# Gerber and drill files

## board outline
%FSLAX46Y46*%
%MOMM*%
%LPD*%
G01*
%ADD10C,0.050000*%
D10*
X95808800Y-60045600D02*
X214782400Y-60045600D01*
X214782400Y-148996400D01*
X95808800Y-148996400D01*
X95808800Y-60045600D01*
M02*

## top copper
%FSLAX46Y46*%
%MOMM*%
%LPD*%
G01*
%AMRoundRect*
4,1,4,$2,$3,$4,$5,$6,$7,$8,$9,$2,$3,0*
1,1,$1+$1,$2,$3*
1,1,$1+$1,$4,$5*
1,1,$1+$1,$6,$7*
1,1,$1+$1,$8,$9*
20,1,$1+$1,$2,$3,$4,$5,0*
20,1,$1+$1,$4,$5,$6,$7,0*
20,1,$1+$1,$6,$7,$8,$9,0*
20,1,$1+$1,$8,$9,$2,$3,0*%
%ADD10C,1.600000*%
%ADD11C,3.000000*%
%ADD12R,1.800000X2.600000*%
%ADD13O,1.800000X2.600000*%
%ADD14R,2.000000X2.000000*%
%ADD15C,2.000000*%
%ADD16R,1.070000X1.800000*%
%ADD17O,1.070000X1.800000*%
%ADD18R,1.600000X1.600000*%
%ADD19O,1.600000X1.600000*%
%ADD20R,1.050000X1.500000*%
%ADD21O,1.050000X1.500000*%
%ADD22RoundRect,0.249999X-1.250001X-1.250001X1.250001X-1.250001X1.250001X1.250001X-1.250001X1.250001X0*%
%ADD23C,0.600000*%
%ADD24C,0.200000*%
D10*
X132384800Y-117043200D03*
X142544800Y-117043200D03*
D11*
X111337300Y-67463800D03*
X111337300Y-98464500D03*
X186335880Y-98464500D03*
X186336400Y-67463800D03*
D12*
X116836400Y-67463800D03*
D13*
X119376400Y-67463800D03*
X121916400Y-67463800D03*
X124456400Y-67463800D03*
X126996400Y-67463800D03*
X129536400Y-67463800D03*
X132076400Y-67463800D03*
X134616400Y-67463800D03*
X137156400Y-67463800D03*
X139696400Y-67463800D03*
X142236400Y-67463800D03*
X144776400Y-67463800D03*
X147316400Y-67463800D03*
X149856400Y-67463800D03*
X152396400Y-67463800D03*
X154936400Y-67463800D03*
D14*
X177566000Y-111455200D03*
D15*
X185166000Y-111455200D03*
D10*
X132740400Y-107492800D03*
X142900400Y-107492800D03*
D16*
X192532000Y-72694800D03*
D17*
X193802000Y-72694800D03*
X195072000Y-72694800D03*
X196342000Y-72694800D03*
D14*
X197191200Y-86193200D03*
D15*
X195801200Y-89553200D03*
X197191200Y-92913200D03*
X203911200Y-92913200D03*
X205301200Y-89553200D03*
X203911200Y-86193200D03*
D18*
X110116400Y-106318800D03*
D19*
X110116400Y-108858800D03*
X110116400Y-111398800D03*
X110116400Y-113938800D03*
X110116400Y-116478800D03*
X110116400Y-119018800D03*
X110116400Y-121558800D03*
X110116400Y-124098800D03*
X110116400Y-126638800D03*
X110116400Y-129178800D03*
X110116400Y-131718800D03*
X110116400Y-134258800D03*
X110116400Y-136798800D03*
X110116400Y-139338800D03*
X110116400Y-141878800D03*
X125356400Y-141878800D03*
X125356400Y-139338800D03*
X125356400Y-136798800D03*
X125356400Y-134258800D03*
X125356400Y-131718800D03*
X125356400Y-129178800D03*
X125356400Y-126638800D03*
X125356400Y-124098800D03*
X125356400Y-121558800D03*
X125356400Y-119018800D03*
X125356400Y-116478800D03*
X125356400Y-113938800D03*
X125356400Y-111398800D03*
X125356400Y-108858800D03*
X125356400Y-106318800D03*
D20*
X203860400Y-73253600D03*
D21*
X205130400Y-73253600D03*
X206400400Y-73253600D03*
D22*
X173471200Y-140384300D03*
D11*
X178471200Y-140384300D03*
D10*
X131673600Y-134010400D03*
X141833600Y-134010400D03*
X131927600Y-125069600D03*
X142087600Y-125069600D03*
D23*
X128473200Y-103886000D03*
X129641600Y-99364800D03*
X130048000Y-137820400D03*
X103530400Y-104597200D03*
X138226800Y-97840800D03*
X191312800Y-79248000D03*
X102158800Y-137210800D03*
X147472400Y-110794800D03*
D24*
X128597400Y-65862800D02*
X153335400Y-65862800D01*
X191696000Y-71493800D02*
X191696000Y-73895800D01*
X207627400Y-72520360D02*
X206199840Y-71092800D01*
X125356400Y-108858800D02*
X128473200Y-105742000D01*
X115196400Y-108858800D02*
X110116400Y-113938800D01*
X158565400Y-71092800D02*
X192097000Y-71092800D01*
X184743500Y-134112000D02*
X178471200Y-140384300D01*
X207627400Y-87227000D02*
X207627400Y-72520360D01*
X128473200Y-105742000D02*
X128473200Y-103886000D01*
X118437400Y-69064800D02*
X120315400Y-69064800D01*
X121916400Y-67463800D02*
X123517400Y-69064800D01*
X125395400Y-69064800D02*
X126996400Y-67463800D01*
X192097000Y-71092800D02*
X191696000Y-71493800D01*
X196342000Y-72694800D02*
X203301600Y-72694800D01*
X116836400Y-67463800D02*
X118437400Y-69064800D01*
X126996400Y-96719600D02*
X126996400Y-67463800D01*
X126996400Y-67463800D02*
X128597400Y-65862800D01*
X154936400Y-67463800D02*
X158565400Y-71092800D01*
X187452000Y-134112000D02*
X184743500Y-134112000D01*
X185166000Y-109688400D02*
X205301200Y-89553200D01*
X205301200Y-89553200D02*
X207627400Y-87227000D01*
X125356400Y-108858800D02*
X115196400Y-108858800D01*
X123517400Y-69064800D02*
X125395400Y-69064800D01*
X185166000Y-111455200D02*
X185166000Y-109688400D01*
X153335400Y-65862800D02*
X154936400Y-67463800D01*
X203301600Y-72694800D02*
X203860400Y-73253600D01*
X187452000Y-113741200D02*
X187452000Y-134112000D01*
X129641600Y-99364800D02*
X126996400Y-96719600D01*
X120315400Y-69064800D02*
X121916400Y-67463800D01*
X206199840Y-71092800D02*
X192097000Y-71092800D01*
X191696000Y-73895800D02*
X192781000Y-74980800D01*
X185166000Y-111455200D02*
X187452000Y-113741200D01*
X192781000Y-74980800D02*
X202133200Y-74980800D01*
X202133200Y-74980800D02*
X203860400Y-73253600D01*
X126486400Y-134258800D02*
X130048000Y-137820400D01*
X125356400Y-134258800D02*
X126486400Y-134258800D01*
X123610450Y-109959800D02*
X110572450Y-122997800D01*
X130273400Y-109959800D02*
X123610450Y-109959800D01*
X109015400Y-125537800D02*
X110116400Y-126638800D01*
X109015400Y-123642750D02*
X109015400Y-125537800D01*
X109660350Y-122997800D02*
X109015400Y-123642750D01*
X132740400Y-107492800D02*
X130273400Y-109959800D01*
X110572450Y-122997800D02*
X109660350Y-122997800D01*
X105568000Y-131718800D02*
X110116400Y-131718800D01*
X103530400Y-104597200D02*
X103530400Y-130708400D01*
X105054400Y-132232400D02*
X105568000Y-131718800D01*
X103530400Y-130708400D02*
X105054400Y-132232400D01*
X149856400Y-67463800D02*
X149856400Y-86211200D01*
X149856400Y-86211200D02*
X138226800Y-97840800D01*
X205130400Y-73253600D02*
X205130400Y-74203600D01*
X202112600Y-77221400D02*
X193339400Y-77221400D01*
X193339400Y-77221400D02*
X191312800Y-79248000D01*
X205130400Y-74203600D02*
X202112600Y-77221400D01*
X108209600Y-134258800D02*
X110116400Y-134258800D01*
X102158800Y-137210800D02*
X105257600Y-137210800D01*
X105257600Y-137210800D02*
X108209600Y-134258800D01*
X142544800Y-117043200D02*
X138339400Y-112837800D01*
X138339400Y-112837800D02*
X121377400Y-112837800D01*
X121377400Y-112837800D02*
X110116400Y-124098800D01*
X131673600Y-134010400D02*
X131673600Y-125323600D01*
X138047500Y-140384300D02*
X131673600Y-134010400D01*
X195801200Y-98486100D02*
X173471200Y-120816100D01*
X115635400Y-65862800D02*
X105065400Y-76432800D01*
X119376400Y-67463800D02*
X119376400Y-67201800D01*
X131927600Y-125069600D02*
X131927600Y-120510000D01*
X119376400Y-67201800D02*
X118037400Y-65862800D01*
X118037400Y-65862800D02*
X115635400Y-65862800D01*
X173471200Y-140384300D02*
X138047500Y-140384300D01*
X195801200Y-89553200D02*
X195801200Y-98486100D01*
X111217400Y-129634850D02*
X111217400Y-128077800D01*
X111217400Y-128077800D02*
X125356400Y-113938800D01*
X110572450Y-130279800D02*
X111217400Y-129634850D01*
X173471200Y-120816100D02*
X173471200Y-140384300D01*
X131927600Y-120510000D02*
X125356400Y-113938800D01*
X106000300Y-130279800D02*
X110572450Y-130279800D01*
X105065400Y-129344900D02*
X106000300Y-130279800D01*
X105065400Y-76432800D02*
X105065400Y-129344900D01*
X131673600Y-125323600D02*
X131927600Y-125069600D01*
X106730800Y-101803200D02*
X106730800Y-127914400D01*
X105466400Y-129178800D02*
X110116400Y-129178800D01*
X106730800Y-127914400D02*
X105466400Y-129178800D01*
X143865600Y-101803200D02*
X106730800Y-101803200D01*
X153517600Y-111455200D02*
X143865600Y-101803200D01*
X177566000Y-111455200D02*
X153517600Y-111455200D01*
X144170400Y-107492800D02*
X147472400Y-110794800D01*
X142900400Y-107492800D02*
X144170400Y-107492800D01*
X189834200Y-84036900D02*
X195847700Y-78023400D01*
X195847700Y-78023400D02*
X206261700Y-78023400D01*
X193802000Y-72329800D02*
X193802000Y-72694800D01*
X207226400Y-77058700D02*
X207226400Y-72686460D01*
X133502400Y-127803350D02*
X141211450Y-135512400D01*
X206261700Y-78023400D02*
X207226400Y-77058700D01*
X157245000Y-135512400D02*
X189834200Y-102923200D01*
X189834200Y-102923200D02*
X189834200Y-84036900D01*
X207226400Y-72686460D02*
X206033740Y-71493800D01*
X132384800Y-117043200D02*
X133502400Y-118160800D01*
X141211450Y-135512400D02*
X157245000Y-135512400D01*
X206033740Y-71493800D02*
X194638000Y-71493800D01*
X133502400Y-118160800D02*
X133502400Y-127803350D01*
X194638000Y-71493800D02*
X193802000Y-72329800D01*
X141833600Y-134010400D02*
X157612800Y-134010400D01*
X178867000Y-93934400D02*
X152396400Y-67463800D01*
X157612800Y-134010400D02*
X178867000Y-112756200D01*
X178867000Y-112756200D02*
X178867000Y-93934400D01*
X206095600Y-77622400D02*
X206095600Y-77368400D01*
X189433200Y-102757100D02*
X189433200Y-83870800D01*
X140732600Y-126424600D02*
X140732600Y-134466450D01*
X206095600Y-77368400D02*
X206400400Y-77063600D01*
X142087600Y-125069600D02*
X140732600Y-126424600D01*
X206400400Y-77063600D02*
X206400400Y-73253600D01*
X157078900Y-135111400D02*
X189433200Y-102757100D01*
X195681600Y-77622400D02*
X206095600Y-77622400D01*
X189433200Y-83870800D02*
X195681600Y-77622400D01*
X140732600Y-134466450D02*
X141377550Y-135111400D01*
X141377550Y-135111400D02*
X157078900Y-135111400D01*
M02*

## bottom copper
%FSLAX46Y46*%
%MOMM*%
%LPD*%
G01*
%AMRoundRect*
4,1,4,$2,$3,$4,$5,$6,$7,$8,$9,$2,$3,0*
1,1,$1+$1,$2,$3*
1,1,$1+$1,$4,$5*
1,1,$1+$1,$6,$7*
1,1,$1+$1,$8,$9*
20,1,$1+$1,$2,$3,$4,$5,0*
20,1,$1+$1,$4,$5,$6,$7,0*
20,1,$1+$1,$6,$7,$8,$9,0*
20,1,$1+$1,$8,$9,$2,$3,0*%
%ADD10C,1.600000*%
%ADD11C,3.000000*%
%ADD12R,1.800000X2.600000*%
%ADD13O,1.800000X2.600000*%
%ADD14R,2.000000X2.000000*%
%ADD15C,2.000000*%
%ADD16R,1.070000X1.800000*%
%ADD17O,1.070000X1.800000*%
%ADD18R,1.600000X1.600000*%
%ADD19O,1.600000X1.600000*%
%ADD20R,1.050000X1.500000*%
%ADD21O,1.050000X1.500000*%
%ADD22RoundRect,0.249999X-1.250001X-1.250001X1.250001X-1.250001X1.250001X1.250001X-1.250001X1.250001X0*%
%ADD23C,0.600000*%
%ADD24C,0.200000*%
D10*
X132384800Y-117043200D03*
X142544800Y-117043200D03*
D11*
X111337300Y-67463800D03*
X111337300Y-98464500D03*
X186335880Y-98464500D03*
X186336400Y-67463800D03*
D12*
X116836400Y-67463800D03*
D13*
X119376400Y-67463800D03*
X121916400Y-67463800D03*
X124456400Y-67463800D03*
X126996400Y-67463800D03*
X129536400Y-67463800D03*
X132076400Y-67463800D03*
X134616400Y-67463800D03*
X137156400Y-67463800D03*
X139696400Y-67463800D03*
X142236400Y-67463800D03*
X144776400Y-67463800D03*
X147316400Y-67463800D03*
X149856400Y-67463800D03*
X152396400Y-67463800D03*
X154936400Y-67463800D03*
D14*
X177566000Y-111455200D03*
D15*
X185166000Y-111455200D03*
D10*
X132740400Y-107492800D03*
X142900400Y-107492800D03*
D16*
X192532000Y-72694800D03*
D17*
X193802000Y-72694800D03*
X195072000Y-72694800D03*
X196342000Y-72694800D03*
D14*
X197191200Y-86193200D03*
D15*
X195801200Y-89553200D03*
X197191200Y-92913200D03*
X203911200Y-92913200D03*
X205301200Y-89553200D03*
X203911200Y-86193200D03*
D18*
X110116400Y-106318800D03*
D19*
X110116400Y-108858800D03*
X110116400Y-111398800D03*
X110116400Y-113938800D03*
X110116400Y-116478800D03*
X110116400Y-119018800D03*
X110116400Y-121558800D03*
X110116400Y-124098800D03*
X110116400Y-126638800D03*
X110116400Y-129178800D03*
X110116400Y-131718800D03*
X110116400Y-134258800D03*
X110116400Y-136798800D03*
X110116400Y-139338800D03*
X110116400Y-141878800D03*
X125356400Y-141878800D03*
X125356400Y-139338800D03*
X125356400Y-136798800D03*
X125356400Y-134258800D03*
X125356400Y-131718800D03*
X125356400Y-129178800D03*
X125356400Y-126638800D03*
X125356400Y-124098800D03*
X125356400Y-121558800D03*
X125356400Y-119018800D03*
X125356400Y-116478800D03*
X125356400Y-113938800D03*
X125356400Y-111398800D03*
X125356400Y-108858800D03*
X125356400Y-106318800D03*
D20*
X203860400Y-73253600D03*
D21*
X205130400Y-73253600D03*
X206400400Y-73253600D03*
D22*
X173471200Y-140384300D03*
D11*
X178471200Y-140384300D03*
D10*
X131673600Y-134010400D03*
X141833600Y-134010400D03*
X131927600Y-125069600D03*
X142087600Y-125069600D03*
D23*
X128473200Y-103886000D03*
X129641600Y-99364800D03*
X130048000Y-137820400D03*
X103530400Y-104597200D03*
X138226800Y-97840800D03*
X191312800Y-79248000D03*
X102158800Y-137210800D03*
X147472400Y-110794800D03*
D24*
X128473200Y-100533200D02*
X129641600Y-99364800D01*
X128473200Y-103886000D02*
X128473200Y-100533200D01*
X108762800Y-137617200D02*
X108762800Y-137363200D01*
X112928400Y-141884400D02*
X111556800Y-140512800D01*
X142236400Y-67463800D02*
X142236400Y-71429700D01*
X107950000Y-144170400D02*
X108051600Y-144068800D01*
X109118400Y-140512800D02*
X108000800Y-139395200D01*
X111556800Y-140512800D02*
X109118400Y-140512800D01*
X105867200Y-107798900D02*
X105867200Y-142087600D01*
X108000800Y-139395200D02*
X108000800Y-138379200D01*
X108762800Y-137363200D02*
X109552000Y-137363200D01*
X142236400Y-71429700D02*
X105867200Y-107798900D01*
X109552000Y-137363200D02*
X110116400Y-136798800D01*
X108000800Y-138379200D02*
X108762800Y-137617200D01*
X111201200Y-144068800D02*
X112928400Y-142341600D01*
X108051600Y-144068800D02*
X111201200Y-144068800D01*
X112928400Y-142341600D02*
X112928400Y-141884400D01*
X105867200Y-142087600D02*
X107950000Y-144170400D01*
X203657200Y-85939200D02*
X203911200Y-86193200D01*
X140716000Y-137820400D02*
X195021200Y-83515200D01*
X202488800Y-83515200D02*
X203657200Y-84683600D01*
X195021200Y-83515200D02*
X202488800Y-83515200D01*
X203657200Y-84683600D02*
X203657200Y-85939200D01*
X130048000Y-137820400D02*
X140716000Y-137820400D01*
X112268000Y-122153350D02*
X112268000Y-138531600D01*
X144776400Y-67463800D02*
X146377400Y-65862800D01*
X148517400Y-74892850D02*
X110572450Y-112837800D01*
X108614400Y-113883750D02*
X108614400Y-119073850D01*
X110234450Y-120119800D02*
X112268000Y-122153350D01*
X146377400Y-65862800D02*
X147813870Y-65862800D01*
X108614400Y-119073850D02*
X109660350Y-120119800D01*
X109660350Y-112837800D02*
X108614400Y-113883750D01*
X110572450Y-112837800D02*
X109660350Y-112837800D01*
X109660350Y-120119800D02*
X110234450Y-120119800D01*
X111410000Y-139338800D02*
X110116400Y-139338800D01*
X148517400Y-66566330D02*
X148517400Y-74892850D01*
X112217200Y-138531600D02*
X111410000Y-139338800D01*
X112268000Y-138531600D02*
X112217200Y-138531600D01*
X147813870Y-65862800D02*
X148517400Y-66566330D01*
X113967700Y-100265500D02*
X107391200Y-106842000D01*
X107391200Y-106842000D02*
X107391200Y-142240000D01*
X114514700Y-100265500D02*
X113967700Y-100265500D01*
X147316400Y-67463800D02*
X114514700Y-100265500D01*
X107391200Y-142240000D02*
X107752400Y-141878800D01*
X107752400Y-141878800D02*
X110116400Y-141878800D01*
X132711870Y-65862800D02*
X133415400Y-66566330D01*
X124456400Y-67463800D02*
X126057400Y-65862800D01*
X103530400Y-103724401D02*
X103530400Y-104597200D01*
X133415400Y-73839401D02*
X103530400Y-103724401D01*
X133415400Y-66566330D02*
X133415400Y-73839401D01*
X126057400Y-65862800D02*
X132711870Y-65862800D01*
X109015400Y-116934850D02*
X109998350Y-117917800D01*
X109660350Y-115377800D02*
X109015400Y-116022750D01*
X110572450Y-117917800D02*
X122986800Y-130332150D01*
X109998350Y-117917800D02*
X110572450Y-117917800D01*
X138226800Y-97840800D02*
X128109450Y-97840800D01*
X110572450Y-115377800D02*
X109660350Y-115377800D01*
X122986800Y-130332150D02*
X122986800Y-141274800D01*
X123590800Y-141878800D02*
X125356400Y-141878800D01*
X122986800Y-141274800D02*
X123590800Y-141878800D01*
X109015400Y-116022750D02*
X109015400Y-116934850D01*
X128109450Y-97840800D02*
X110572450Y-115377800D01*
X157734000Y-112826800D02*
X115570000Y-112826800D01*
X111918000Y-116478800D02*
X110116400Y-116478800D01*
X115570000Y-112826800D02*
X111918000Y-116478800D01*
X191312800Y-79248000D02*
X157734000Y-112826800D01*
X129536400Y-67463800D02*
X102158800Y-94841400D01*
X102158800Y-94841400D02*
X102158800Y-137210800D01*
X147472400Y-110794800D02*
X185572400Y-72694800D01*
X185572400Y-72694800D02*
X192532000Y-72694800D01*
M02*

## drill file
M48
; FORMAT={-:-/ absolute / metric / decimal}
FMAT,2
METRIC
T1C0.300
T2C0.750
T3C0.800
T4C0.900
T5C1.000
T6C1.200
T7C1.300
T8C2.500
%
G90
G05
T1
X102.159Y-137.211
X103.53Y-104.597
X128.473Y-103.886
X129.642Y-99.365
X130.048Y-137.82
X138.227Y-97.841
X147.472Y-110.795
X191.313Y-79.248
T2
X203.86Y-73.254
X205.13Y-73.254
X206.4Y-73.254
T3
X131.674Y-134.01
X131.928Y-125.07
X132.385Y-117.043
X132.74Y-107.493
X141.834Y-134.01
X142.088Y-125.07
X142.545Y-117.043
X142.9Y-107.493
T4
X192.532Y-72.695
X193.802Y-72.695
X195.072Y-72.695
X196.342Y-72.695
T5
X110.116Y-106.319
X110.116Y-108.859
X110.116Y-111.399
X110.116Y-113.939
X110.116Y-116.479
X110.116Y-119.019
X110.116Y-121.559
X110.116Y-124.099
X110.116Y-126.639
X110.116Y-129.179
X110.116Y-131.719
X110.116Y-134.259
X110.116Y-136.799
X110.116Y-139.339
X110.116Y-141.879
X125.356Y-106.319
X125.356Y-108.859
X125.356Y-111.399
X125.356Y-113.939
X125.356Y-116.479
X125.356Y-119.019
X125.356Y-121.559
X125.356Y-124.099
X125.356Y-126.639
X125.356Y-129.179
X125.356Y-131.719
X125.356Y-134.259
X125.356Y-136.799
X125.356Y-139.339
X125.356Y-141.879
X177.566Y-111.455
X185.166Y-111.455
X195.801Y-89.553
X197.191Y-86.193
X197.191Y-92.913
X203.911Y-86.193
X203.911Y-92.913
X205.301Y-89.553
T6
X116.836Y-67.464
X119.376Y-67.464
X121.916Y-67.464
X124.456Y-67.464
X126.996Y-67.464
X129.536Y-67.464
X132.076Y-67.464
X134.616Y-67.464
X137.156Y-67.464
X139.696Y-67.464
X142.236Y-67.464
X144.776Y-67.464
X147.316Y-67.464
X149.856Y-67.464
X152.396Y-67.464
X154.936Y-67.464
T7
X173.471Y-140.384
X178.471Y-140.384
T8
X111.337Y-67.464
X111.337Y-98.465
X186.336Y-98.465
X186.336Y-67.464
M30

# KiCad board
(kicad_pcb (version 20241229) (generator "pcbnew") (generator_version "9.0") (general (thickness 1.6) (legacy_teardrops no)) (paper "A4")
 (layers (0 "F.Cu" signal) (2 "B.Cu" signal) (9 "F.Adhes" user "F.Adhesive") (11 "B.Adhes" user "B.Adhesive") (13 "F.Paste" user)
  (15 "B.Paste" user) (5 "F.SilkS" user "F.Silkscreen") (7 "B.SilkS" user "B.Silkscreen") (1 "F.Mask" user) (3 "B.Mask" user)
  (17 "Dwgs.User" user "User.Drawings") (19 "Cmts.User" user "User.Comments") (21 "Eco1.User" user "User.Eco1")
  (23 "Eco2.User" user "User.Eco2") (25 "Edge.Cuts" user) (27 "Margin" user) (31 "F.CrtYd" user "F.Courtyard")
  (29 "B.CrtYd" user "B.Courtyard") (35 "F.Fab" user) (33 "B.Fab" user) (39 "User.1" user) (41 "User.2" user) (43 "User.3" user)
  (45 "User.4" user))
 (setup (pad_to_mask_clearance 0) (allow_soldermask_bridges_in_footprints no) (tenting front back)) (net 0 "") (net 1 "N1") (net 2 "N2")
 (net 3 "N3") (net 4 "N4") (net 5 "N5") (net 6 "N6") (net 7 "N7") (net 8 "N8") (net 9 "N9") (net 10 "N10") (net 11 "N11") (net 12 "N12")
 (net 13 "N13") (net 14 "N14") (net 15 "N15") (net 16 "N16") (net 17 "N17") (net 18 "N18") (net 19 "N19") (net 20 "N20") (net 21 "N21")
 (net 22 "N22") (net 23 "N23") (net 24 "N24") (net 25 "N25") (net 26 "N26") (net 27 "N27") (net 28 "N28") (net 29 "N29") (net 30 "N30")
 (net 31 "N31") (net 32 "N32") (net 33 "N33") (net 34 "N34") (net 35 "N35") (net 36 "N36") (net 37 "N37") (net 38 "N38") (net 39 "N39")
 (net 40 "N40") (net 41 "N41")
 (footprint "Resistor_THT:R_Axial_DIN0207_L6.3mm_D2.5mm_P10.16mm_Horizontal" (layer "F.Cu") (at 132.3848 117.0432)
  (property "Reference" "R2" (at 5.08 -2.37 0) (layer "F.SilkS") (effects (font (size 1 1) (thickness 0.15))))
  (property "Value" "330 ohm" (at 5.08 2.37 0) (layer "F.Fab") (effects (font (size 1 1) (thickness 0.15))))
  (pad "1" thru_hole circle (at 0 0) (size 1.6 1.6) (drill 0.8) (layers "*.Cu" "*.Mask") (remove_unused_layers no) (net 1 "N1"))
  (pad "2" thru_hole circle (at 10.16 0) (size 1.6 1.6) (drill 0.8) (layers "*.Cu" "*.Mask") (remove_unused_layers no) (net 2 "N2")))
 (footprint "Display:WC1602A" (layer "F.Cu") (at 116.8364 67.4638)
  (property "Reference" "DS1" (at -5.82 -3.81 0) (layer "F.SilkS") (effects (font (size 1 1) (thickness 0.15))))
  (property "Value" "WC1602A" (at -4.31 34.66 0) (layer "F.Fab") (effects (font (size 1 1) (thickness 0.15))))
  (pad "" thru_hole circle (at -5.4991 0) (size 3 3) (drill 2.5) (layers "*.Cu" "*.Mask") (remove_unused_layers no))
  (pad "" thru_hole circle (at -5.4991 31.0007) (size 3 3) (drill 2.5) (layers "*.Cu" "*.Mask") (remove_unused_layers no))
  (pad "" thru_hole circle (at 69.49948 31.0007) (size 3 3) (drill 2.5) (layers "*.Cu" "*.Mask") (remove_unused_layers no))
  (pad "" thru_hole circle (at 69.5 0) (size 3 3) (drill 2.5) (layers "*.Cu" "*.Mask") (remove_unused_layers no))
  (pad "1" thru_hole rect (at 0 0) (size 1.8 2.6) (drill 1.2) (layers "*.Cu" "*.Mask") (remove_unused_layers no) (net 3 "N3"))
  (pad "2" thru_hole oval (at 2.54 0) (size 1.8 2.6) (drill 1.2) (layers "*.Cu" "*.Mask") (remove_unused_layers no) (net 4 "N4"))
  (pad "3" thru_hole oval (at 5.08 0) (size 1.8 2.6) (drill 1.2) (layers "*.Cu" "*.Mask") (remove_unused_layers no) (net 3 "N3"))
  (pad "4" thru_hole oval (at 7.62 0) (size 1.8 2.6) (drill 1.2) (layers "*.Cu" "*.Mask") (remove_unused_layers no) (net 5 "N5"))
  (pad "5" thru_hole oval (at 10.16 0) (size 1.8 2.6) (drill 1.2) (layers "*.Cu" "*.Mask") (remove_unused_layers no) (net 3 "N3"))
  (pad "6" thru_hole oval (at 12.7 0) (size 1.8 2.6) (drill 1.2) (layers "*.Cu" "*.Mask") (remove_unused_layers no) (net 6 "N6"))
  (pad "7" thru_hole oval (at 15.24 0) (size 1.8 2.6) (drill 1.2) (layers "*.Cu" "*.Mask") (remove_unused_layers no) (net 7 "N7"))
  (pad "8" thru_hole oval (at 17.78 0) (size 1.8 2.6) (drill 1.2) (layers "*.Cu" "*.Mask") (remove_unused_layers no) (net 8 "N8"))
  (pad "9" thru_hole oval (at 20.32 0) (size 1.8 2.6) (drill 1.2) (layers "*.Cu" "*.Mask") (remove_unused_layers no) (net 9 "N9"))
  (pad "10" thru_hole oval (at 22.86 0) (size 1.8 2.6) (drill 1.2) (layers "*.Cu" "*.Mask") (remove_unused_layers no) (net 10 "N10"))
  (pad "11" thru_hole oval (at 25.4 0) (size 1.8 2.6) (drill 1.2) (layers "*.Cu" "*.Mask") (remove_unused_layers no) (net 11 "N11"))
  (pad "12" thru_hole oval (at 27.94 0) (size 1.8 2.6) (drill 1.2) (layers "*.Cu" "*.Mask") (remove_unused_layers no) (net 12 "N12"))
  (pad "13" thru_hole oval (at 30.48 0) (size 1.8 2.6) (drill 1.2) (layers "*.Cu" "*.Mask") (remove_unused_layers no) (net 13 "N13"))
  (pad "14" thru_hole oval (at 33.02 0) (size 1.8 2.6) (drill 1.2) (layers "*.Cu" "*.Mask") (remove_unused_layers no) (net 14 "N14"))
  (pad "15" thru_hole oval (at 35.56 0) (size 1.8 2.6) (drill 1.2) (layers "*.Cu" "*.Mask") (remove_unused_layers no) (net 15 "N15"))
  (pad "16" thru_hole oval (at 38.1 0) (size 1.8 2.6) (drill 1.2) (layers "*.Cu" "*.Mask") (remove_unused_layers no) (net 3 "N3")))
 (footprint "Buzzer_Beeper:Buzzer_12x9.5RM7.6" (layer "F.Cu") (at 177.566 111.4552)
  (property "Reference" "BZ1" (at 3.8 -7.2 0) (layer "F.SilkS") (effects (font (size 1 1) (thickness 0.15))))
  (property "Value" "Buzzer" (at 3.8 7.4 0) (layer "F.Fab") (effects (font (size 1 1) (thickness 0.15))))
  (pad "1" thru_hole rect (at 0 0) (size 2 2) (drill 1) (layers "*.Cu" "*.Mask") (remove_unused_layers no) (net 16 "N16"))
  (pad "2" thru_hole circle (at 7.6 0) (size 2 2) (drill 1) (layers "*.Cu" "*.Mask") (remove_unused_layers no) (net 3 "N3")))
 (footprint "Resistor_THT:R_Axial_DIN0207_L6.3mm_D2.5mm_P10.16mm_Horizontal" (layer "F.Cu") (at 132.7404 107.4928)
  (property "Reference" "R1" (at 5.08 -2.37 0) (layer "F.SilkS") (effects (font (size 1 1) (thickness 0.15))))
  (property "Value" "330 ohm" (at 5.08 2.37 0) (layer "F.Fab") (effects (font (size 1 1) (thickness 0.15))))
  (pad "1" thru_hole circle (at 0 0) (size 1.6 1.6) (drill 0.8) (layers "*.Cu" "*.Mask") (remove_unused_layers no) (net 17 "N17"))
  (pad "2" thru_hole circle (at 10.16 0) (size 1.6 1.6) (drill 0.8) (layers "*.Cu" "*.Mask") (remove_unused_layers no) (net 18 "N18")))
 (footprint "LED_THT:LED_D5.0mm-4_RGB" (layer "F.Cu") (at 192.532 72.6948)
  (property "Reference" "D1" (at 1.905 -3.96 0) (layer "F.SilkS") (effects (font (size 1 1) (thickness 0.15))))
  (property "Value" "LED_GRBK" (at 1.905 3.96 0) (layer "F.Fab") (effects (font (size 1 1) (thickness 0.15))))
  (pad "1" thru_hole rect (at 0 0) (size 1.07 1.8) (drill 0.9) (layers "*.Cu" "*.Mask") (remove_unused_layers no) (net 18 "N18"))
  (pad "2" thru_hole oval (at 1.27 0) (size 1.07 1.8) (drill 0.9) (layers "*.Cu" "*.Mask") (remove_unused_layers no) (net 1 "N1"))
  (pad "3" thru_hole oval (at 2.54 0) (size 1.07 1.8) (drill 0.9) (layers "*.Cu" "*.Mask") (remove_unused_layers no) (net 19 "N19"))
  (pad "4" thru_hole oval (at 3.81 0) (size 1.07 1.8) (drill 0.9) (layers "*.Cu" "*.Mask") (remove_unused_layers no) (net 3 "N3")))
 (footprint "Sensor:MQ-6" (layer "F.Cu") (at 197.1912 86.1932)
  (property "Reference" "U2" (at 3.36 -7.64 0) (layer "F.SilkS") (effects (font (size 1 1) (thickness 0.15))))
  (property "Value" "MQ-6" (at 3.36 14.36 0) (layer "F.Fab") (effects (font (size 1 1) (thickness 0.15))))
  (pad "1" thru_hole rect (at 0 0) (size 2 2) (drill 1) (layers "*.Cu" "*.Mask") (remove_unused_layers no) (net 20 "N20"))
  (pad "2" thru_hole circle (at -1.39 3.36) (size 2 2) (drill 1) (layers "*.Cu" "*.Mask") (remove_unused_layers no) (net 4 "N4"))
  (pad "3" thru_hole circle (at 0 6.72 90) (size 2 2) (drill 1) (layers "*.Cu" "*.Mask") (remove_unused_layers no) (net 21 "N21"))
  (pad "4" thru_hole circle (at 6.72 6.72 180) (size 2 2) (drill 1) (layers "*.Cu" "*.Mask") (remove_unused_layers no) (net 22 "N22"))
  (pad "5" thru_hole circle (at 8.11 3.36) (size 2 2) (drill 1) (layers "*.Cu" "*.Mask") (remove_unused_layers no) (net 3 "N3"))
  (pad "6" thru_hole circle (at 6.72 0 270) (size 2 2) (drill 1) (layers "*.Cu" "*.Mask") (remove_unused_layers no) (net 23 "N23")))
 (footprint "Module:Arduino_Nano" (layer "F.Cu") (at 110.1164 106.3188)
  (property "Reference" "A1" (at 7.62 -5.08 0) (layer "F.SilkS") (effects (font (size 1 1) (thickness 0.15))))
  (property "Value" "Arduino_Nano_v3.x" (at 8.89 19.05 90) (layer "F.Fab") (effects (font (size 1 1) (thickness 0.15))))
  (pad "1" thru_hole rect (at 0 0) (size 1.6 1.6) (drill 1) (layers "*.Cu" "*.Mask") (remove_unused_layers no) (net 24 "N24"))
  (pad "2" thru_hole oval (at 0 2.54) (size 1.6 1.6) (drill 1) (layers "*.Cu" "*.Mask") (remove_unused_layers no) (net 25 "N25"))
  (pad "3" thru_hole oval (at 0 5.08) (size 1.6 1.6) (drill 1) (layers "*.Cu" "*.Mask") (remove_unused_layers no) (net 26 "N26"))
  (pad "4" thru_hole oval (at 0 7.62) (size 1.6 1.6) (drill 1) (layers "*.Cu" "*.Mask") (remove_unused_layers no) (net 3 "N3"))
  (pad "5" thru_hole oval (at 0 10.16) (size 1.6 1.6) (drill 1) (layers "*.Cu" "*.Mask") (remove_unused_layers no) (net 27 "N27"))
  (pad "6" thru_hole oval (at 0 12.7) (size 1.6 1.6) (drill 1) (layers "*.Cu" "*.Mask") (remove_unused_layers no) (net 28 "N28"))
  (pad "7" thru_hole oval (at 0 15.24) (size 1.6 1.6) (drill 1) (layers "*.Cu" "*.Mask") (remove_unused_layers no) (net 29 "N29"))
  (pad "8" thru_hole oval (at 0 17.78) (size 1.6 1.6) (drill 1) (layers "*.Cu" "*.Mask") (remove_unused_layers no) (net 2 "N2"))
  (pad "9" thru_hole oval (at 0 20.32) (size 1.6 1.6) (drill 1) (layers "*.Cu" "*.Mask") (remove_unused_layers no) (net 17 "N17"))
  (pad "10" thru_hole oval (at 0 22.86) (size 1.6 1.6) (drill 1) (layers "*.Cu" "*.Mask") (remove_unused_layers no) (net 16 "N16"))
  (pad "11" thru_hole oval (at 0 25.4) (size 1.6 1.6) (drill 1) (layers "*.Cu" "*.Mask") (remove_unused_layers no) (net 5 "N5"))
  (pad "12" thru_hole oval (at 0 27.94) (size 1.6 1.6) (drill 1) (layers "*.Cu" "*.Mask") (remove_unused_layers no) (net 6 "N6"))
  (pad "13" thru_hole oval (at 0 30.48) (size 1.6 1.6) (drill 1) (layers "*.Cu" "*.Mask") (remove_unused_layers no) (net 11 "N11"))
  (pad "14" thru_hole oval (at 0 33.02) (size 1.6 1.6) (drill 1) (layers "*.Cu" "*.Mask") (remove_unused_layers no) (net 12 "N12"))
  (pad "15" thru_hole oval (at 0 35.56) (size 1.6 1.6) (drill 1) (layers "*.Cu" "*.Mask") (remove_unused_layers no) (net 13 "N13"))
  (pad "16" thru_hole oval (at 15.24 35.56) (size 1.6 1.6) (drill 1) (layers "*.Cu" "*.Mask") (remove_unused_layers no) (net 14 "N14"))
  (pad "17" thru_hole oval (at 15.24 33.02) (size 1.6 1.6) (drill 1) (layers "*.Cu" "*.Mask") (remove_unused_layers no) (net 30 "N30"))
  (pad "18" thru_hole oval (at 15.24 30.48) (size 1.6 1.6) (drill 1) (layers "*.Cu" "*.Mask") (remove_unused_layers no) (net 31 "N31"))
  (pad "19" thru_hole oval (at 15.24 27.94) (size 1.6 1.6) (drill 1) (layers "*.Cu" "*.Mask") (remove_unused_layers no) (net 23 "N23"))
  (pad "20" thru_hole oval (at 15.24 25.4) (size 1.6 1.6) (drill 1) (layers "*.Cu" "*.Mask") (remove_unused_layers no) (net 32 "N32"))
  (pad "21" thru_hole oval (at 15.24 22.86) (size 1.6 1.6) (drill 1) (layers "*.Cu" "*.Mask") (remove_unused_layers no) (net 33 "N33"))
  (pad "22" thru_hole oval (at 15.24 20.32) (size 1.6 1.6) (drill 1) (layers "*.Cu" "*.Mask") (remove_unused_layers no) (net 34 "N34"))
  (pad "23" thru_hole oval (at 15.24 17.78) (size 1.6 1.6) (drill 1) (layers "*.Cu" "*.Mask") (remove_unused_layers no) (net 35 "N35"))
  (pad "24" thru_hole oval (at 15.24 15.24) (size 1.6 1.6) (drill 1) (layers "*.Cu" "*.Mask") (remove_unused_layers no) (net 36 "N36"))
  (pad "25" thru_hole oval (at 15.24 12.7) (size 1.6 1.6) (drill 1) (layers "*.Cu" "*.Mask") (remove_unused_layers no) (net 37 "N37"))
  (pad "26" thru_hole oval (at 15.24 10.16) (size 1.6 1.6) (drill 1) (layers "*.Cu" "*.Mask") (remove_unused_layers no) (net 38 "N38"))
  (pad "27" thru_hole oval (at 15.24 7.62) (size 1.6 1.6) (drill 1) (layers "*.Cu" "*.Mask") (remove_unused_layers no) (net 4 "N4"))
  (pad "28" thru_hole oval (at 15.24 5.08) (size 1.6 1.6) (drill 1) (layers "*.Cu" "*.Mask") (remove_unused_layers no) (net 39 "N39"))
  (pad "29" thru_hole oval (at 15.24 2.54) (size 1.6 1.6) (drill 1) (layers "*.Cu" "*.Mask") (remove_unused_layers no) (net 3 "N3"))
  (pad "30" thru_hole oval (at 15.24 0) (size 1.6 1.6) (drill 1) (layers "*.Cu" "*.Mask") (remove_unused_layers no) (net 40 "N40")))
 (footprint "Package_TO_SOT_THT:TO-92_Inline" (layer "F.Cu") (at 203.8604 73.2536)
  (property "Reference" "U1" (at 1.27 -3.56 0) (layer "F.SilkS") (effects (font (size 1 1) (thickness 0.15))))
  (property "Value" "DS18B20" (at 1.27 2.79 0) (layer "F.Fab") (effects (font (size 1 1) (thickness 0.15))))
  (pad "1" thru_hole rect (at 0 0) (size 1.05 1.5) (drill 0.75) (layers "*.Cu" "*.Mask") (remove_unused_layers no) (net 3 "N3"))
  (pad "2" thru_hole oval (at 1.27 0) (size 1.05 1.5) (drill 0.75) (layers "*.Cu" "*.Mask") (remove_unused_layers no) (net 27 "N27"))
  (pad "3" thru_hole oval (at 2.54 0) (size 1.05 1.5) (drill 0.75) (layers "*.Cu" "*.Mask") (remove_unused_layers no) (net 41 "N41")))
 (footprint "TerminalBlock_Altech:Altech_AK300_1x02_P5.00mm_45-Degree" (layer "F.Cu") (at 173.4712 140.3843)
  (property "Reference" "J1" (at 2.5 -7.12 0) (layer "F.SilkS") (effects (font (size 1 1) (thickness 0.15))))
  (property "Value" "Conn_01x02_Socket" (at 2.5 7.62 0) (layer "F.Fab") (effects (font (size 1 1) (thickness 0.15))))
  (pad "1" thru_hole roundrect (at 0 0) (size 3 3) (drill 1.3) (layers "*.Cu" "*.Mask") (remove_unused_layers no)
   (roundrect_rratio 0.083333) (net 4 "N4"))
  (pad "2" thru_hole circle (at 5 0) (size 3 3) (drill 1.3) (layers "*.Cu" "*.Mask") (remove_unused_layers no) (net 3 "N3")))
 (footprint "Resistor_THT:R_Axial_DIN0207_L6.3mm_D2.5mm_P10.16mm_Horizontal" (layer "F.Cu") (at 131.6736 134.0104)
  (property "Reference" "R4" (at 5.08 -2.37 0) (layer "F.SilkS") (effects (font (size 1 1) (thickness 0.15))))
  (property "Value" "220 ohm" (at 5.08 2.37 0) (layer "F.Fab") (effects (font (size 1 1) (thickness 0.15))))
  (pad "1" thru_hole circle (at 0 0) (size 1.6 1.6) (drill 0.8) (layers "*.Cu" "*.Mask") (remove_unused_layers no) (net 4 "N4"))
  (pad "2" thru_hole circle (at 10.16 0) (size 1.6 1.6) (drill 0.8) (layers "*.Cu" "*.Mask") (remove_unused_layers no) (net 15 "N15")))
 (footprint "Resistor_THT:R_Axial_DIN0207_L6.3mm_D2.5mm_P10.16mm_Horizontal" (layer "F.Cu") (at 131.9276 125.0696)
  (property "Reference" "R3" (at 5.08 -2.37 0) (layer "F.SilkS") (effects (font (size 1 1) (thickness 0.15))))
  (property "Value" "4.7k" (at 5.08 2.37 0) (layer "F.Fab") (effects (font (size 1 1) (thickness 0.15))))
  (pad "1" thru_hole circle (at 0 0) (size 1.6 1.6) (drill 0.8) (layers "*.Cu" "*.Mask") (remove_unused_layers no) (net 4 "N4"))
  (pad "2" thru_hole circle (at 10.16 0) (size 1.6 1.6) (drill 0.8) (layers "*.Cu" "*.Mask") (remove_unused_layers no) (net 41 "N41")))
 (gr_rect (start 95.8088 60.0456) (end 214.7824 148.9964) (stroke (width 0.05) (type default)) (fill no) (layer "Edge.Cuts"))
 (segment (start 128.5974 65.8628) (end 153.3354 65.8628) (width 0.2) (layer "F.Cu") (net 3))
 (segment (start 191.696 71.4938) (end 191.696 73.8958) (width 0.2) (layer "F.Cu") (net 3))
 (segment (start 207.6274 72.52036) (end 206.19984 71.0928) (width 0.2) (layer "F.Cu") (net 3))
 (segment (start 125.3564 108.8588) (end 128.4732 105.742) (width 0.2) (layer "F.Cu") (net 3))
 (segment (start 115.1964 108.8588) (end 110.1164 113.9388) (width 0.2) (layer "F.Cu") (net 3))
 (segment (start 158.5654 71.0928) (end 192.097 71.0928) (width 0.2) (layer "F.Cu") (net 3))
 (segment (start 184.7435 134.112) (end 178.4712 140.3843) (width 0.2) (layer "F.Cu") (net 3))
 (segment (start 207.6274 87.227) (end 207.6274 72.52036) (width 0.2) (layer "F.Cu") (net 3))
 (segment (start 128.4732 105.742) (end 128.4732 103.886) (width 0.2) (layer "F.Cu") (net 3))
 (segment (start 118.4374 69.0648) (end 120.3154 69.0648) (width 0.2) (layer "F.Cu") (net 3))
 (segment (start 121.9164 67.4638) (end 123.5174 69.0648) (width 0.2) (layer "F.Cu") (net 3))
 (segment (start 125.3954 69.0648) (end 126.9964 67.4638) (width 0.2) (layer "F.Cu") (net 3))
 (segment (start 192.097 71.0928) (end 191.696 71.4938) (width 0.2) (layer "F.Cu") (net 3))
 (segment (start 196.342 72.6948) (end 203.3016 72.6948) (width 0.2) (layer "F.Cu") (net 3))
 (segment (start 116.8364 67.4638) (end 118.4374 69.0648) (width 0.2) (layer "F.Cu") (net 3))
 (segment (start 126.9964 96.7196) (end 126.9964 67.4638) (width 0.2) (layer "F.Cu") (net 3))
 (segment (start 126.9964 67.4638) (end 128.5974 65.8628) (width 0.2) (layer "F.Cu") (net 3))
 (segment (start 154.9364 67.4638) (end 158.5654 71.0928) (width 0.2) (layer "F.Cu") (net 3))
 (segment (start 187.452 134.112) (end 184.7435 134.112) (width 0.2) (layer "F.Cu") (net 3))
 (segment (start 185.166 109.6884) (end 205.3012 89.5532) (width 0.2) (layer "F.Cu") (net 3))
 (segment (start 205.3012 89.5532) (end 207.6274 87.227) (width 0.2) (layer "F.Cu") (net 3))
 (segment (start 125.3564 108.8588) (end 115.1964 108.8588) (width 0.2) (layer "F.Cu") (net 3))
 (segment (start 123.5174 69.0648) (end 125.3954 69.0648) (width 0.2) (layer "F.Cu") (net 3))
 (segment (start 185.166 111.4552) (end 185.166 109.6884) (width 0.2) (layer "F.Cu") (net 3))
 (segment (start 153.3354 65.8628) (end 154.9364 67.4638) (width 0.2) (layer "F.Cu") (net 3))
 (segment (start 203.3016 72.6948) (end 203.8604 73.2536) (width 0.2) (layer "F.Cu") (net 3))
 (segment (start 187.452 113.7412) (end 187.452 134.112) (width 0.2) (layer "F.Cu") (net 3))
 (segment (start 129.6416 99.3648) (end 126.9964 96.7196) (width 0.2) (layer "F.Cu") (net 3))
 (segment (start 120.3154 69.0648) (end 121.9164 67.4638) (width 0.2) (layer "F.Cu") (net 3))
 (segment (start 206.19984 71.0928) (end 192.097 71.0928) (width 0.2) (layer "F.Cu") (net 3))
 (segment (start 191.696 73.8958) (end 192.781 74.9808) (width 0.2) (layer "F.Cu") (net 3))
 (segment (start 185.166 111.4552) (end 187.452 113.7412) (width 0.2) (layer "F.Cu") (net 3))
 (segment (start 192.781 74.9808) (end 202.1332 74.9808) (width 0.2) (layer "F.Cu") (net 3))
 (segment (start 202.1332 74.9808) (end 203.8604 73.2536) (width 0.2) (layer "F.Cu") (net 3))
 (via (at 128.4732 103.886) (size 0.6) (drill 0.3) (layers "F.Cu" "B.Cu") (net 3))
 (via (at 129.6416 99.3648) (size 0.6) (drill 0.3) (layers "F.Cu" "B.Cu") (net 3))
 (segment (start 128.4732 100.5332) (end 129.6416 99.3648) (width 0.2) (layer "B.Cu") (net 3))
 (segment (start 128.4732 103.886) (end 128.4732 100.5332) (width 0.2) (layer "B.Cu") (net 3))
 (segment (start 108.7628 137.6172) (end 108.7628 137.3632) (width 0.2) (layer "B.Cu") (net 11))
 (segment (start 112.9284 141.8844) (end 111.5568 140.5128) (width 0.2) (layer "B.Cu") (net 11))
 (segment (start 142.2364 67.4638) (end 142.2364 71.4297) (width 0.2) (layer "B.Cu") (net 11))
 (segment (start 107.95 144.1704) (end 108.0516 144.0688) (width 0.2) (layer "B.Cu") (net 11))
 (segment (start 109.1184 140.5128) (end 108.0008 139.3952) (width 0.2) (layer "B.Cu") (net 11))
 (segment (start 111.5568 140.5128) (end 109.1184 140.5128) (width 0.2) (layer "B.Cu") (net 11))
 (segment (start 105.8672 107.7989) (end 105.8672 142.0876) (width 0.2) (layer "B.Cu") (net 11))
 (segment (start 108.0008 139.3952) (end 108.0008 138.3792) (width 0.2) (layer "B.Cu") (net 11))
 (segment (start 108.7628 137.3632) (end 109.552 137.3632) (width 0.2) (layer "B.Cu") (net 11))
 (segment (start 142.2364 71.4297) (end 105.8672 107.7989) (width 0.2) (layer "B.Cu") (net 11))
 (segment (start 109.552 137.3632) (end 110.1164 136.7988) (width 0.2) (layer "B.Cu") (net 11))
 (segment (start 108.0008 138.3792) (end 108.7628 137.6172) (width 0.2) (layer "B.Cu") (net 11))
 (segment (start 111.2012 144.0688) (end 112.9284 142.3416) (width 0.2) (layer "B.Cu") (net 11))
 (segment (start 108.0516 144.0688) (end 111.2012 144.0688) (width 0.2) (layer "B.Cu") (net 11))
 (segment (start 112.9284 142.3416) (end 112.9284 141.8844) (width 0.2) (layer "B.Cu") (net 11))
 (segment (start 105.8672 142.0876) (end 107.95 144.1704) (width 0.2) (layer "B.Cu") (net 11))
 (segment (start 126.4864 134.2588) (end 130.048 137.8204) (width 0.2) (layer "F.Cu") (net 23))
 (segment (start 125.3564 134.2588) (end 126.4864 134.2588) (width 0.2) (layer "F.Cu") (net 23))
 (via (at 130.048 137.8204) (size 0.6) (drill 0.3) (layers "F.Cu" "B.Cu") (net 23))
 (segment (start 203.6572 85.9392) (end 203.9112 86.1932) (width 0.2) (layer "B.Cu") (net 23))
 (segment (start 140.716 137.8204) (end 195.0212 83.5152) (width 0.2) (layer "B.Cu") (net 23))
 (segment (start 202.4888 83.5152) (end 203.6572 84.6836) (width 0.2) (layer "B.Cu") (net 23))
 (segment (start 195.0212 83.5152) (end 202.4888 83.5152) (width 0.2) (layer "B.Cu") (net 23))
 (segment (start 203.6572 84.6836) (end 203.6572 85.9392) (width 0.2) (layer "B.Cu") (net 23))
 (segment (start 130.048 137.8204) (end 140.716 137.8204) (width 0.2) (layer "B.Cu") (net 23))
 (segment (start 112.268 122.15335) (end 112.268 138.5316) (width 0.2) (layer "B.Cu") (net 12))
 (segment (start 144.7764 67.4638) (end 146.3774 65.8628) (width 0.2) (layer "B.Cu") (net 12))
 (segment (start 148.5174 74.89285) (end 110.57245 112.8378) (width 0.2) (layer "B.Cu") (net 12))
 (segment (start 108.6144 113.88375) (end 108.6144 119.07385) (width 0.2) (layer "B.Cu") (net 12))
 (segment (start 110.23445 120.1198) (end 112.268 122.15335) (width 0.2) (layer "B.Cu") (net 12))
 (segment (start 146.3774 65.8628) (end 147.81387 65.8628) (width 0.2) (layer "B.Cu") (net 12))
 (segment (start 108.6144 119.07385) (end 109.66035 120.1198) (width 0.2) (layer "B.Cu") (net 12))
 (segment (start 109.66035 112.8378) (end 108.6144 113.88375) (width 0.2) (layer "B.Cu") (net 12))
 (segment (start 110.57245 112.8378) (end 109.66035 112.8378) (width 0.2) (layer "B.Cu") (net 12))
 (segment (start 109.66035 120.1198) (end 110.23445 120.1198) (width 0.2) (layer "B.Cu") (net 12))
 (segment (start 111.41 139.3388) (end 110.1164 139.3388) (width 0.2) (layer "B.Cu") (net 12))
 (segment (start 148.5174 66.56633) (end 148.5174 74.89285) (width 0.2) (layer "B.Cu") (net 12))
 (segment (start 112.2172 138.5316) (end 111.41 139.3388) (width 0.2) (layer "B.Cu") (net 12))
 (segment (start 112.268 138.5316) (end 112.2172 138.5316) (width 0.2) (layer "B.Cu") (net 12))
 (segment (start 147.81387 65.8628) (end 148.5174 66.56633) (width 0.2) (layer "B.Cu") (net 12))
 (segment (start 123.61045 109.9598) (end 110.57245 122.9978) (width 0.2) (layer "F.Cu") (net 17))
 (segment (start 130.2734 109.9598) (end 123.61045 109.9598) (width 0.2) (layer "F.Cu") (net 17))
 (segment (start 109.0154 125.5378) (end 110.1164 126.6388) (width 0.2) (layer "F.Cu") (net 17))
 (segment (start 109.0154 123.64275) (end 109.0154 125.5378) (width 0.2) (layer "F.Cu") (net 17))
 (segment (start 109.66035 122.9978) (end 109.0154 123.64275) (width 0.2) (layer "F.Cu") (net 17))
 (segment (start 132.7404 107.4928) (end 130.2734 109.9598) (width 0.2) (layer "F.Cu") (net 17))
 (segment (start 110.57245 122.9978) (end 109.66035 122.9978) (width 0.2) (layer "F.Cu") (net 17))
 (segment (start 113.9677 100.2655) (end 107.3912 106.842) (width 0.2) (layer "B.Cu") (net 13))
 (segment (start 107.3912 106.842) (end 107.3912 142.24) (width 0.2) (layer "B.Cu") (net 13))
 (segment (start 114.5147 100.2655) (end 113.9677 100.2655) (width 0.2) (layer "B.Cu") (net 13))
 (segment (start 147.3164 67.4638) (end 114.5147 100.2655) (width 0.2) (layer "B.Cu") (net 13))
 (segment (start 107.3912 142.24) (end 107.7524 141.8788) (width 0.2) (layer "B.Cu") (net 13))
 (segment (start 107.7524 141.8788) (end 110.1164 141.8788) (width 0.2) (layer "B.Cu") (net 13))
 (segment (start 105.568 131.7188) (end 110.1164 131.7188) (width 0.2) (layer "F.Cu") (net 5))
 (segment (start 103.5304 104.5972) (end 103.5304 130.7084) (width 0.2) (layer "F.Cu") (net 5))
 (segment (start 105.0544 132.2324) (end 105.568 131.7188) (width 0.2) (layer "F.Cu") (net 5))
 (segment (start 103.5304 130.7084) (end 105.0544 132.2324) (width 0.2) (layer "F.Cu") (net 5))
 (via (at 103.5304 104.5972) (size 0.6) (drill 0.3) (layers "F.Cu" "B.Cu") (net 5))
 (segment (start 132.71187 65.8628) (end 133.4154 66.56633) (width 0.2) (layer "B.Cu") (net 5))
 (segment (start 124.4564 67.4638) (end 126.0574 65.8628) (width 0.2) (layer "B.Cu") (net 5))
 (segment (start 103.5304 103.724401) (end 103.5304 104.5972) (width 0.2) (layer "B.Cu") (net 5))
 (segment (start 133.4154 73.839401) (end 103.5304 103.724401) (width 0.2) (layer "B.Cu") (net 5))
 (segment (start 133.4154 66.56633) (end 133.4154 73.839401) (width 0.2) (layer "B.Cu") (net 5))
 (segment (start 126.0574 65.8628) (end 132.71187 65.8628) (width 0.2) (layer "B.Cu") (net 5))
 (segment (start 149.8564 67.4638) (end 149.8564 86.2112) (width 0.2) (layer "F.Cu") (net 14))
 (segment (start 149.8564 86.2112) (end 138.2268 97.8408) (width 0.2) (layer "F.Cu") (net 14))
 (via (at 138.2268 97.8408) (size 0.6) (drill 0.3) (layers "F.Cu" "B.Cu") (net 14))
 (segment (start 109.0154 116.93485) (end 109.99835 117.9178) (width 0.2) (layer "B.Cu") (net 14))
 (segment (start 109.66035 115.3778) (end 109.0154 116.02275) (width 0.2) (layer "B.Cu") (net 14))
 (segment (start 110.57245 117.9178) (end 122.9868 130.33215) (width 0.2) (layer "B.Cu") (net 14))
 (segment (start 109.99835 117.9178) (end 110.57245 117.9178) (width 0.2) (layer "B.Cu") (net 14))
 (segment (start 138.2268 97.8408) (end 128.10945 97.8408) (width 0.2) (layer "B.Cu") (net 14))
 (segment (start 110.57245 115.3778) (end 109.66035 115.3778) (width 0.2) (layer "B.Cu") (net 14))
 (segment (start 122.9868 130.33215) (end 122.9868 141.2748) (width 0.2) (layer "B.Cu") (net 14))
 (segment (start 123.5908 141.8788) (end 125.3564 141.8788) (width 0.2) (layer "B.Cu") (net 14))
 (segment (start 122.9868 141.2748) (end 123.5908 141.8788) (width 0.2) (layer "B.Cu") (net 14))
 (segment (start 109.0154 116.02275) (end 109.0154 116.93485) (width 0.2) (layer "B.Cu") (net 14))
 (segment (start 128.10945 97.8408) (end 110.57245 115.3778) (width 0.2) (layer "B.Cu") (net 14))
 (segment (start 205.1304 73.2536) (end 205.1304 74.2036) (width 0.2) (layer "F.Cu") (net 27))
 (segment (start 202.1126 77.2214) (end 193.3394 77.2214) (width 0.2) (layer "F.Cu") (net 27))
 (segment (start 193.3394 77.2214) (end 191.3128 79.248) (width 0.2) (layer "F.Cu") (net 27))
 (segment (start 205.1304 74.2036) (end 202.1126 77.2214) (width 0.2) (layer "F.Cu") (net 27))
 (via (at 191.3128 79.248) (size 0.6) (drill 0.3) (layers "F.Cu" "B.Cu") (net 27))
 (segment (start 157.734 112.8268) (end 115.57 112.8268) (width 0.2) (layer "B.Cu") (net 27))
 (segment (start 111.918 116.4788) (end 110.1164 116.4788) (width 0.2) (layer "B.Cu") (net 27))
 (segment (start 115.57 112.8268) (end 111.918 116.4788) (width 0.2) (layer "B.Cu") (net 27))
 (segment (start 191.3128 79.248) (end 157.734 112.8268) (width 0.2) (layer "B.Cu") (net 27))
 (segment (start 108.2096 134.2588) (end 110.1164 134.2588) (width 0.2) (layer "F.Cu") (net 6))
 (segment (start 102.1588 137.2108) (end 105.2576 137.2108) (width 0.2) (layer "F.Cu") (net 6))
 (segment (start 105.2576 137.2108) (end 108.2096 134.2588) (width 0.2) (layer "F.Cu") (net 6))
 (via (at 102.1588 137.2108) (size 0.6) (drill 0.3) (layers "F.Cu" "B.Cu") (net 6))
 (segment (start 129.5364 67.4638) (end 102.1588 94.8414) (width 0.2) (layer "B.Cu") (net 6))
 (segment (start 102.1588 94.8414) (end 102.1588 137.2108) (width 0.2) (layer "B.Cu") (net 6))
 (segment (start 142.5448 117.0432) (end 138.3394 112.8378) (width 0.2) (layer "F.Cu") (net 2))
 (segment (start 138.3394 112.8378) (end 121.3774 112.8378) (width 0.2) (layer "F.Cu") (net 2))
 (segment (start 121.3774 112.8378) (end 110.1164 124.0988) (width 0.2) (layer "F.Cu") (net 2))
 (segment (start 131.6736 134.0104) (end 131.6736 125.3236) (width 0.2) (layer "F.Cu") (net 4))
 (segment (start 138.0475 140.3843) (end 131.6736 134.0104) (width 0.2) (layer "F.Cu") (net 4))
 (segment (start 195.8012 98.4861) (end 173.4712 120.8161) (width 0.2) (layer "F.Cu") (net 4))
 (segment (start 115.6354 65.8628) (end 105.0654 76.4328) (width 0.2) (layer "F.Cu") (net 4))
 (segment (start 119.3764 67.4638) (end 119.3764 67.2018) (width 0.2) (layer "F.Cu") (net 4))
 (segment (start 131.9276 125.0696) (end 131.9276 120.51) (width 0.2) (layer "F.Cu") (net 4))
 (segment (start 119.3764 67.2018) (end 118.0374 65.8628) (width 0.2) (layer "F.Cu") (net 4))
 (segment (start 118.0374 65.8628) (end 115.6354 65.8628) (width 0.2) (layer "F.Cu") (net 4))
 (segment (start 173.4712 140.3843) (end 138.0475 140.3843) (width 0.2) (layer "F.Cu") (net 4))
 (segment (start 195.8012 89.5532) (end 195.8012 98.4861) (width 0.2) (layer "F.Cu") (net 4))
 (segment (start 111.2174 129.63485) (end 111.2174 128.0778) (width 0.2) (layer "F.Cu") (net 4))
 (segment (start 111.2174 128.0778) (end 125.3564 113.9388) (width 0.2) (layer "F.Cu") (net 4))
 (segment (start 110.57245 130.2798) (end 111.2174 129.63485) (width 0.2) (layer "F.Cu") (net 4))
 (segment (start 173.4712 120.8161) (end 173.4712 140.3843) (width 0.2) (layer "F.Cu") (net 4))
 (segment (start 131.9276 120.51) (end 125.3564 113.9388) (width 0.2) (layer "F.Cu") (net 4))
 (segment (start 106.0003 130.2798) (end 110.57245 130.2798) (width 0.2) (layer "F.Cu") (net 4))
 (segment (start 105.0654 129.3449) (end 106.0003 130.2798) (width 0.2) (layer "F.Cu") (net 4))
 (segment (start 105.0654 76.4328) (end 105.0654 129.3449) (width 0.2) (layer "F.Cu") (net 4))
 (segment (start 131.6736 125.3236) (end 131.9276 125.0696) (width 0.2) (layer "F.Cu") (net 4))
 (segment (start 106.7308 101.8032) (end 106.7308 127.9144) (width 0.2) (layer "F.Cu") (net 16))
 (segment (start 105.4664 129.1788) (end 110.1164 129.1788) (width 0.2) (layer "F.Cu") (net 16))
 (segment (start 106.7308 127.9144) (end 105.4664 129.1788) (width 0.2) (layer "F.Cu") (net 16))
 (segment (start 143.8656 101.8032) (end 106.7308 101.8032) (width 0.2) (layer "F.Cu") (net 16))
 (segment (start 153.5176 111.4552) (end 143.8656 101.8032) (width 0.2) (layer "F.Cu") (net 16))
 (segment (start 177.566 111.4552) (end 153.5176 111.4552) (width 0.2) (layer "F.Cu") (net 16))
 (segment (start 144.1704 107.4928) (end 147.4724 110.7948) (width 0.2) (layer "F.Cu") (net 18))
 (segment (start 142.9004 107.4928) (end 144.1704 107.4928) (width 0.2) (layer "F.Cu") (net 18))
 (via (at 147.4724 110.7948) (size 0.6) (drill 0.3) (layers "F.Cu" "B.Cu") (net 18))
 (segment (start 147.4724 110.7948) (end 185.5724 72.6948) (width 0.2) (layer "B.Cu") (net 18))
 (segment (start 185.5724 72.6948) (end 192.532 72.6948) (width 0.2) (layer "B.Cu") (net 18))
 (segment (start 189.8342 84.0369) (end 195.8477 78.0234) (width 0.2) (layer "F.Cu") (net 1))
 (segment (start 195.8477 78.0234) (end 206.2617 78.0234) (width 0.2) (layer "F.Cu") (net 1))
 (segment (start 193.802 72.3298) (end 193.802 72.6948) (width 0.2) (layer "F.Cu") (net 1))
 (segment (start 207.2264 77.0587) (end 207.2264 72.68646) (width 0.2) (layer "F.Cu") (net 1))
 (segment (start 133.5024 127.80335) (end 141.21145 135.5124) (width 0.2) (layer "F.Cu") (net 1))
 (segment (start 206.2617 78.0234) (end 207.2264 77.0587) (width 0.2) (layer "F.Cu") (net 1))
 (segment (start 157.245 135.5124) (end 189.8342 102.9232) (width 0.2) (layer "F.Cu") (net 1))
 (segment (start 189.8342 102.9232) (end 189.8342 84.0369) (width 0.2) (layer "F.Cu") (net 1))
 (segment (start 207.2264 72.68646) (end 206.03374 71.4938) (width 0.2) (layer "F.Cu") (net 1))
 (segment (start 132.3848 117.0432) (end 133.5024 118.1608) (width 0.2) (layer "F.Cu") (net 1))
 (segment (start 141.21145 135.5124) (end 157.245 135.5124) (width 0.2) (layer "F.Cu") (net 1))
 (segment (start 206.03374 71.4938) (end 194.638 71.4938) (width 0.2) (layer "F.Cu") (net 1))
 (segment (start 133.5024 118.1608) (end 133.5024 127.80335) (width 0.2) (layer "F.Cu") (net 1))
 (segment (start 194.638 71.4938) (end 193.802 72.3298) (width 0.2) (layer "F.Cu") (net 1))
 (segment (start 141.8336 134.0104) (end 157.6128 134.0104) (width 0.2) (layer "F.Cu") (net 15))
 (segment (start 178.867 93.9344) (end 152.3964 67.4638) (width 0.2) (layer "F.Cu") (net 15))
 (segment (start 157.6128 134.0104) (end 178.867 112.7562) (width 0.2) (layer "F.Cu") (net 15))
 (segment (start 178.867 112.7562) (end 178.867 93.9344) (width 0.2) (layer "F.Cu") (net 15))
 (segment (start 206.0956 77.6224) (end 206.0956 77.3684) (width 0.2) (layer "F.Cu") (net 41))
 (segment (start 189.4332 102.7571) (end 189.4332 83.8708) (width 0.2) (layer "F.Cu") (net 41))
 (segment (start 140.7326 126.4246) (end 140.7326 134.46645) (width 0.2) (layer "F.Cu") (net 41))
 (segment (start 206.0956 77.3684) (end 206.4004 77.0636) (width 0.2) (layer "F.Cu") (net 41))
 (segment (start 142.0876 125.0696) (end 140.7326 126.4246) (width 0.2) (layer "F.Cu") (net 41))
 (segment (start 206.4004 77.0636) (end 206.4004 73.2536) (width 0.2) (layer "F.Cu") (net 41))
 (segment (start 157.0789 135.1114) (end 189.4332 102.7571) (width 0.2) (layer "F.Cu") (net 41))
 (segment (start 195.6816 77.6224) (end 206.0956 77.6224) (width 0.2) (layer "F.Cu") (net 41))
 (segment (start 189.4332 83.8708) (end 195.6816 77.6224) (width 0.2) (layer "F.Cu") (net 41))
 (segment (start 140.7326 134.46645) (end 141.37755 135.1114) (width 0.2) (layer "F.Cu") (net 41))
 (segment (start 141.37755 135.1114) (end 157.0789 135.1114) (width 0.2) (layer "F.Cu") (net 41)))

